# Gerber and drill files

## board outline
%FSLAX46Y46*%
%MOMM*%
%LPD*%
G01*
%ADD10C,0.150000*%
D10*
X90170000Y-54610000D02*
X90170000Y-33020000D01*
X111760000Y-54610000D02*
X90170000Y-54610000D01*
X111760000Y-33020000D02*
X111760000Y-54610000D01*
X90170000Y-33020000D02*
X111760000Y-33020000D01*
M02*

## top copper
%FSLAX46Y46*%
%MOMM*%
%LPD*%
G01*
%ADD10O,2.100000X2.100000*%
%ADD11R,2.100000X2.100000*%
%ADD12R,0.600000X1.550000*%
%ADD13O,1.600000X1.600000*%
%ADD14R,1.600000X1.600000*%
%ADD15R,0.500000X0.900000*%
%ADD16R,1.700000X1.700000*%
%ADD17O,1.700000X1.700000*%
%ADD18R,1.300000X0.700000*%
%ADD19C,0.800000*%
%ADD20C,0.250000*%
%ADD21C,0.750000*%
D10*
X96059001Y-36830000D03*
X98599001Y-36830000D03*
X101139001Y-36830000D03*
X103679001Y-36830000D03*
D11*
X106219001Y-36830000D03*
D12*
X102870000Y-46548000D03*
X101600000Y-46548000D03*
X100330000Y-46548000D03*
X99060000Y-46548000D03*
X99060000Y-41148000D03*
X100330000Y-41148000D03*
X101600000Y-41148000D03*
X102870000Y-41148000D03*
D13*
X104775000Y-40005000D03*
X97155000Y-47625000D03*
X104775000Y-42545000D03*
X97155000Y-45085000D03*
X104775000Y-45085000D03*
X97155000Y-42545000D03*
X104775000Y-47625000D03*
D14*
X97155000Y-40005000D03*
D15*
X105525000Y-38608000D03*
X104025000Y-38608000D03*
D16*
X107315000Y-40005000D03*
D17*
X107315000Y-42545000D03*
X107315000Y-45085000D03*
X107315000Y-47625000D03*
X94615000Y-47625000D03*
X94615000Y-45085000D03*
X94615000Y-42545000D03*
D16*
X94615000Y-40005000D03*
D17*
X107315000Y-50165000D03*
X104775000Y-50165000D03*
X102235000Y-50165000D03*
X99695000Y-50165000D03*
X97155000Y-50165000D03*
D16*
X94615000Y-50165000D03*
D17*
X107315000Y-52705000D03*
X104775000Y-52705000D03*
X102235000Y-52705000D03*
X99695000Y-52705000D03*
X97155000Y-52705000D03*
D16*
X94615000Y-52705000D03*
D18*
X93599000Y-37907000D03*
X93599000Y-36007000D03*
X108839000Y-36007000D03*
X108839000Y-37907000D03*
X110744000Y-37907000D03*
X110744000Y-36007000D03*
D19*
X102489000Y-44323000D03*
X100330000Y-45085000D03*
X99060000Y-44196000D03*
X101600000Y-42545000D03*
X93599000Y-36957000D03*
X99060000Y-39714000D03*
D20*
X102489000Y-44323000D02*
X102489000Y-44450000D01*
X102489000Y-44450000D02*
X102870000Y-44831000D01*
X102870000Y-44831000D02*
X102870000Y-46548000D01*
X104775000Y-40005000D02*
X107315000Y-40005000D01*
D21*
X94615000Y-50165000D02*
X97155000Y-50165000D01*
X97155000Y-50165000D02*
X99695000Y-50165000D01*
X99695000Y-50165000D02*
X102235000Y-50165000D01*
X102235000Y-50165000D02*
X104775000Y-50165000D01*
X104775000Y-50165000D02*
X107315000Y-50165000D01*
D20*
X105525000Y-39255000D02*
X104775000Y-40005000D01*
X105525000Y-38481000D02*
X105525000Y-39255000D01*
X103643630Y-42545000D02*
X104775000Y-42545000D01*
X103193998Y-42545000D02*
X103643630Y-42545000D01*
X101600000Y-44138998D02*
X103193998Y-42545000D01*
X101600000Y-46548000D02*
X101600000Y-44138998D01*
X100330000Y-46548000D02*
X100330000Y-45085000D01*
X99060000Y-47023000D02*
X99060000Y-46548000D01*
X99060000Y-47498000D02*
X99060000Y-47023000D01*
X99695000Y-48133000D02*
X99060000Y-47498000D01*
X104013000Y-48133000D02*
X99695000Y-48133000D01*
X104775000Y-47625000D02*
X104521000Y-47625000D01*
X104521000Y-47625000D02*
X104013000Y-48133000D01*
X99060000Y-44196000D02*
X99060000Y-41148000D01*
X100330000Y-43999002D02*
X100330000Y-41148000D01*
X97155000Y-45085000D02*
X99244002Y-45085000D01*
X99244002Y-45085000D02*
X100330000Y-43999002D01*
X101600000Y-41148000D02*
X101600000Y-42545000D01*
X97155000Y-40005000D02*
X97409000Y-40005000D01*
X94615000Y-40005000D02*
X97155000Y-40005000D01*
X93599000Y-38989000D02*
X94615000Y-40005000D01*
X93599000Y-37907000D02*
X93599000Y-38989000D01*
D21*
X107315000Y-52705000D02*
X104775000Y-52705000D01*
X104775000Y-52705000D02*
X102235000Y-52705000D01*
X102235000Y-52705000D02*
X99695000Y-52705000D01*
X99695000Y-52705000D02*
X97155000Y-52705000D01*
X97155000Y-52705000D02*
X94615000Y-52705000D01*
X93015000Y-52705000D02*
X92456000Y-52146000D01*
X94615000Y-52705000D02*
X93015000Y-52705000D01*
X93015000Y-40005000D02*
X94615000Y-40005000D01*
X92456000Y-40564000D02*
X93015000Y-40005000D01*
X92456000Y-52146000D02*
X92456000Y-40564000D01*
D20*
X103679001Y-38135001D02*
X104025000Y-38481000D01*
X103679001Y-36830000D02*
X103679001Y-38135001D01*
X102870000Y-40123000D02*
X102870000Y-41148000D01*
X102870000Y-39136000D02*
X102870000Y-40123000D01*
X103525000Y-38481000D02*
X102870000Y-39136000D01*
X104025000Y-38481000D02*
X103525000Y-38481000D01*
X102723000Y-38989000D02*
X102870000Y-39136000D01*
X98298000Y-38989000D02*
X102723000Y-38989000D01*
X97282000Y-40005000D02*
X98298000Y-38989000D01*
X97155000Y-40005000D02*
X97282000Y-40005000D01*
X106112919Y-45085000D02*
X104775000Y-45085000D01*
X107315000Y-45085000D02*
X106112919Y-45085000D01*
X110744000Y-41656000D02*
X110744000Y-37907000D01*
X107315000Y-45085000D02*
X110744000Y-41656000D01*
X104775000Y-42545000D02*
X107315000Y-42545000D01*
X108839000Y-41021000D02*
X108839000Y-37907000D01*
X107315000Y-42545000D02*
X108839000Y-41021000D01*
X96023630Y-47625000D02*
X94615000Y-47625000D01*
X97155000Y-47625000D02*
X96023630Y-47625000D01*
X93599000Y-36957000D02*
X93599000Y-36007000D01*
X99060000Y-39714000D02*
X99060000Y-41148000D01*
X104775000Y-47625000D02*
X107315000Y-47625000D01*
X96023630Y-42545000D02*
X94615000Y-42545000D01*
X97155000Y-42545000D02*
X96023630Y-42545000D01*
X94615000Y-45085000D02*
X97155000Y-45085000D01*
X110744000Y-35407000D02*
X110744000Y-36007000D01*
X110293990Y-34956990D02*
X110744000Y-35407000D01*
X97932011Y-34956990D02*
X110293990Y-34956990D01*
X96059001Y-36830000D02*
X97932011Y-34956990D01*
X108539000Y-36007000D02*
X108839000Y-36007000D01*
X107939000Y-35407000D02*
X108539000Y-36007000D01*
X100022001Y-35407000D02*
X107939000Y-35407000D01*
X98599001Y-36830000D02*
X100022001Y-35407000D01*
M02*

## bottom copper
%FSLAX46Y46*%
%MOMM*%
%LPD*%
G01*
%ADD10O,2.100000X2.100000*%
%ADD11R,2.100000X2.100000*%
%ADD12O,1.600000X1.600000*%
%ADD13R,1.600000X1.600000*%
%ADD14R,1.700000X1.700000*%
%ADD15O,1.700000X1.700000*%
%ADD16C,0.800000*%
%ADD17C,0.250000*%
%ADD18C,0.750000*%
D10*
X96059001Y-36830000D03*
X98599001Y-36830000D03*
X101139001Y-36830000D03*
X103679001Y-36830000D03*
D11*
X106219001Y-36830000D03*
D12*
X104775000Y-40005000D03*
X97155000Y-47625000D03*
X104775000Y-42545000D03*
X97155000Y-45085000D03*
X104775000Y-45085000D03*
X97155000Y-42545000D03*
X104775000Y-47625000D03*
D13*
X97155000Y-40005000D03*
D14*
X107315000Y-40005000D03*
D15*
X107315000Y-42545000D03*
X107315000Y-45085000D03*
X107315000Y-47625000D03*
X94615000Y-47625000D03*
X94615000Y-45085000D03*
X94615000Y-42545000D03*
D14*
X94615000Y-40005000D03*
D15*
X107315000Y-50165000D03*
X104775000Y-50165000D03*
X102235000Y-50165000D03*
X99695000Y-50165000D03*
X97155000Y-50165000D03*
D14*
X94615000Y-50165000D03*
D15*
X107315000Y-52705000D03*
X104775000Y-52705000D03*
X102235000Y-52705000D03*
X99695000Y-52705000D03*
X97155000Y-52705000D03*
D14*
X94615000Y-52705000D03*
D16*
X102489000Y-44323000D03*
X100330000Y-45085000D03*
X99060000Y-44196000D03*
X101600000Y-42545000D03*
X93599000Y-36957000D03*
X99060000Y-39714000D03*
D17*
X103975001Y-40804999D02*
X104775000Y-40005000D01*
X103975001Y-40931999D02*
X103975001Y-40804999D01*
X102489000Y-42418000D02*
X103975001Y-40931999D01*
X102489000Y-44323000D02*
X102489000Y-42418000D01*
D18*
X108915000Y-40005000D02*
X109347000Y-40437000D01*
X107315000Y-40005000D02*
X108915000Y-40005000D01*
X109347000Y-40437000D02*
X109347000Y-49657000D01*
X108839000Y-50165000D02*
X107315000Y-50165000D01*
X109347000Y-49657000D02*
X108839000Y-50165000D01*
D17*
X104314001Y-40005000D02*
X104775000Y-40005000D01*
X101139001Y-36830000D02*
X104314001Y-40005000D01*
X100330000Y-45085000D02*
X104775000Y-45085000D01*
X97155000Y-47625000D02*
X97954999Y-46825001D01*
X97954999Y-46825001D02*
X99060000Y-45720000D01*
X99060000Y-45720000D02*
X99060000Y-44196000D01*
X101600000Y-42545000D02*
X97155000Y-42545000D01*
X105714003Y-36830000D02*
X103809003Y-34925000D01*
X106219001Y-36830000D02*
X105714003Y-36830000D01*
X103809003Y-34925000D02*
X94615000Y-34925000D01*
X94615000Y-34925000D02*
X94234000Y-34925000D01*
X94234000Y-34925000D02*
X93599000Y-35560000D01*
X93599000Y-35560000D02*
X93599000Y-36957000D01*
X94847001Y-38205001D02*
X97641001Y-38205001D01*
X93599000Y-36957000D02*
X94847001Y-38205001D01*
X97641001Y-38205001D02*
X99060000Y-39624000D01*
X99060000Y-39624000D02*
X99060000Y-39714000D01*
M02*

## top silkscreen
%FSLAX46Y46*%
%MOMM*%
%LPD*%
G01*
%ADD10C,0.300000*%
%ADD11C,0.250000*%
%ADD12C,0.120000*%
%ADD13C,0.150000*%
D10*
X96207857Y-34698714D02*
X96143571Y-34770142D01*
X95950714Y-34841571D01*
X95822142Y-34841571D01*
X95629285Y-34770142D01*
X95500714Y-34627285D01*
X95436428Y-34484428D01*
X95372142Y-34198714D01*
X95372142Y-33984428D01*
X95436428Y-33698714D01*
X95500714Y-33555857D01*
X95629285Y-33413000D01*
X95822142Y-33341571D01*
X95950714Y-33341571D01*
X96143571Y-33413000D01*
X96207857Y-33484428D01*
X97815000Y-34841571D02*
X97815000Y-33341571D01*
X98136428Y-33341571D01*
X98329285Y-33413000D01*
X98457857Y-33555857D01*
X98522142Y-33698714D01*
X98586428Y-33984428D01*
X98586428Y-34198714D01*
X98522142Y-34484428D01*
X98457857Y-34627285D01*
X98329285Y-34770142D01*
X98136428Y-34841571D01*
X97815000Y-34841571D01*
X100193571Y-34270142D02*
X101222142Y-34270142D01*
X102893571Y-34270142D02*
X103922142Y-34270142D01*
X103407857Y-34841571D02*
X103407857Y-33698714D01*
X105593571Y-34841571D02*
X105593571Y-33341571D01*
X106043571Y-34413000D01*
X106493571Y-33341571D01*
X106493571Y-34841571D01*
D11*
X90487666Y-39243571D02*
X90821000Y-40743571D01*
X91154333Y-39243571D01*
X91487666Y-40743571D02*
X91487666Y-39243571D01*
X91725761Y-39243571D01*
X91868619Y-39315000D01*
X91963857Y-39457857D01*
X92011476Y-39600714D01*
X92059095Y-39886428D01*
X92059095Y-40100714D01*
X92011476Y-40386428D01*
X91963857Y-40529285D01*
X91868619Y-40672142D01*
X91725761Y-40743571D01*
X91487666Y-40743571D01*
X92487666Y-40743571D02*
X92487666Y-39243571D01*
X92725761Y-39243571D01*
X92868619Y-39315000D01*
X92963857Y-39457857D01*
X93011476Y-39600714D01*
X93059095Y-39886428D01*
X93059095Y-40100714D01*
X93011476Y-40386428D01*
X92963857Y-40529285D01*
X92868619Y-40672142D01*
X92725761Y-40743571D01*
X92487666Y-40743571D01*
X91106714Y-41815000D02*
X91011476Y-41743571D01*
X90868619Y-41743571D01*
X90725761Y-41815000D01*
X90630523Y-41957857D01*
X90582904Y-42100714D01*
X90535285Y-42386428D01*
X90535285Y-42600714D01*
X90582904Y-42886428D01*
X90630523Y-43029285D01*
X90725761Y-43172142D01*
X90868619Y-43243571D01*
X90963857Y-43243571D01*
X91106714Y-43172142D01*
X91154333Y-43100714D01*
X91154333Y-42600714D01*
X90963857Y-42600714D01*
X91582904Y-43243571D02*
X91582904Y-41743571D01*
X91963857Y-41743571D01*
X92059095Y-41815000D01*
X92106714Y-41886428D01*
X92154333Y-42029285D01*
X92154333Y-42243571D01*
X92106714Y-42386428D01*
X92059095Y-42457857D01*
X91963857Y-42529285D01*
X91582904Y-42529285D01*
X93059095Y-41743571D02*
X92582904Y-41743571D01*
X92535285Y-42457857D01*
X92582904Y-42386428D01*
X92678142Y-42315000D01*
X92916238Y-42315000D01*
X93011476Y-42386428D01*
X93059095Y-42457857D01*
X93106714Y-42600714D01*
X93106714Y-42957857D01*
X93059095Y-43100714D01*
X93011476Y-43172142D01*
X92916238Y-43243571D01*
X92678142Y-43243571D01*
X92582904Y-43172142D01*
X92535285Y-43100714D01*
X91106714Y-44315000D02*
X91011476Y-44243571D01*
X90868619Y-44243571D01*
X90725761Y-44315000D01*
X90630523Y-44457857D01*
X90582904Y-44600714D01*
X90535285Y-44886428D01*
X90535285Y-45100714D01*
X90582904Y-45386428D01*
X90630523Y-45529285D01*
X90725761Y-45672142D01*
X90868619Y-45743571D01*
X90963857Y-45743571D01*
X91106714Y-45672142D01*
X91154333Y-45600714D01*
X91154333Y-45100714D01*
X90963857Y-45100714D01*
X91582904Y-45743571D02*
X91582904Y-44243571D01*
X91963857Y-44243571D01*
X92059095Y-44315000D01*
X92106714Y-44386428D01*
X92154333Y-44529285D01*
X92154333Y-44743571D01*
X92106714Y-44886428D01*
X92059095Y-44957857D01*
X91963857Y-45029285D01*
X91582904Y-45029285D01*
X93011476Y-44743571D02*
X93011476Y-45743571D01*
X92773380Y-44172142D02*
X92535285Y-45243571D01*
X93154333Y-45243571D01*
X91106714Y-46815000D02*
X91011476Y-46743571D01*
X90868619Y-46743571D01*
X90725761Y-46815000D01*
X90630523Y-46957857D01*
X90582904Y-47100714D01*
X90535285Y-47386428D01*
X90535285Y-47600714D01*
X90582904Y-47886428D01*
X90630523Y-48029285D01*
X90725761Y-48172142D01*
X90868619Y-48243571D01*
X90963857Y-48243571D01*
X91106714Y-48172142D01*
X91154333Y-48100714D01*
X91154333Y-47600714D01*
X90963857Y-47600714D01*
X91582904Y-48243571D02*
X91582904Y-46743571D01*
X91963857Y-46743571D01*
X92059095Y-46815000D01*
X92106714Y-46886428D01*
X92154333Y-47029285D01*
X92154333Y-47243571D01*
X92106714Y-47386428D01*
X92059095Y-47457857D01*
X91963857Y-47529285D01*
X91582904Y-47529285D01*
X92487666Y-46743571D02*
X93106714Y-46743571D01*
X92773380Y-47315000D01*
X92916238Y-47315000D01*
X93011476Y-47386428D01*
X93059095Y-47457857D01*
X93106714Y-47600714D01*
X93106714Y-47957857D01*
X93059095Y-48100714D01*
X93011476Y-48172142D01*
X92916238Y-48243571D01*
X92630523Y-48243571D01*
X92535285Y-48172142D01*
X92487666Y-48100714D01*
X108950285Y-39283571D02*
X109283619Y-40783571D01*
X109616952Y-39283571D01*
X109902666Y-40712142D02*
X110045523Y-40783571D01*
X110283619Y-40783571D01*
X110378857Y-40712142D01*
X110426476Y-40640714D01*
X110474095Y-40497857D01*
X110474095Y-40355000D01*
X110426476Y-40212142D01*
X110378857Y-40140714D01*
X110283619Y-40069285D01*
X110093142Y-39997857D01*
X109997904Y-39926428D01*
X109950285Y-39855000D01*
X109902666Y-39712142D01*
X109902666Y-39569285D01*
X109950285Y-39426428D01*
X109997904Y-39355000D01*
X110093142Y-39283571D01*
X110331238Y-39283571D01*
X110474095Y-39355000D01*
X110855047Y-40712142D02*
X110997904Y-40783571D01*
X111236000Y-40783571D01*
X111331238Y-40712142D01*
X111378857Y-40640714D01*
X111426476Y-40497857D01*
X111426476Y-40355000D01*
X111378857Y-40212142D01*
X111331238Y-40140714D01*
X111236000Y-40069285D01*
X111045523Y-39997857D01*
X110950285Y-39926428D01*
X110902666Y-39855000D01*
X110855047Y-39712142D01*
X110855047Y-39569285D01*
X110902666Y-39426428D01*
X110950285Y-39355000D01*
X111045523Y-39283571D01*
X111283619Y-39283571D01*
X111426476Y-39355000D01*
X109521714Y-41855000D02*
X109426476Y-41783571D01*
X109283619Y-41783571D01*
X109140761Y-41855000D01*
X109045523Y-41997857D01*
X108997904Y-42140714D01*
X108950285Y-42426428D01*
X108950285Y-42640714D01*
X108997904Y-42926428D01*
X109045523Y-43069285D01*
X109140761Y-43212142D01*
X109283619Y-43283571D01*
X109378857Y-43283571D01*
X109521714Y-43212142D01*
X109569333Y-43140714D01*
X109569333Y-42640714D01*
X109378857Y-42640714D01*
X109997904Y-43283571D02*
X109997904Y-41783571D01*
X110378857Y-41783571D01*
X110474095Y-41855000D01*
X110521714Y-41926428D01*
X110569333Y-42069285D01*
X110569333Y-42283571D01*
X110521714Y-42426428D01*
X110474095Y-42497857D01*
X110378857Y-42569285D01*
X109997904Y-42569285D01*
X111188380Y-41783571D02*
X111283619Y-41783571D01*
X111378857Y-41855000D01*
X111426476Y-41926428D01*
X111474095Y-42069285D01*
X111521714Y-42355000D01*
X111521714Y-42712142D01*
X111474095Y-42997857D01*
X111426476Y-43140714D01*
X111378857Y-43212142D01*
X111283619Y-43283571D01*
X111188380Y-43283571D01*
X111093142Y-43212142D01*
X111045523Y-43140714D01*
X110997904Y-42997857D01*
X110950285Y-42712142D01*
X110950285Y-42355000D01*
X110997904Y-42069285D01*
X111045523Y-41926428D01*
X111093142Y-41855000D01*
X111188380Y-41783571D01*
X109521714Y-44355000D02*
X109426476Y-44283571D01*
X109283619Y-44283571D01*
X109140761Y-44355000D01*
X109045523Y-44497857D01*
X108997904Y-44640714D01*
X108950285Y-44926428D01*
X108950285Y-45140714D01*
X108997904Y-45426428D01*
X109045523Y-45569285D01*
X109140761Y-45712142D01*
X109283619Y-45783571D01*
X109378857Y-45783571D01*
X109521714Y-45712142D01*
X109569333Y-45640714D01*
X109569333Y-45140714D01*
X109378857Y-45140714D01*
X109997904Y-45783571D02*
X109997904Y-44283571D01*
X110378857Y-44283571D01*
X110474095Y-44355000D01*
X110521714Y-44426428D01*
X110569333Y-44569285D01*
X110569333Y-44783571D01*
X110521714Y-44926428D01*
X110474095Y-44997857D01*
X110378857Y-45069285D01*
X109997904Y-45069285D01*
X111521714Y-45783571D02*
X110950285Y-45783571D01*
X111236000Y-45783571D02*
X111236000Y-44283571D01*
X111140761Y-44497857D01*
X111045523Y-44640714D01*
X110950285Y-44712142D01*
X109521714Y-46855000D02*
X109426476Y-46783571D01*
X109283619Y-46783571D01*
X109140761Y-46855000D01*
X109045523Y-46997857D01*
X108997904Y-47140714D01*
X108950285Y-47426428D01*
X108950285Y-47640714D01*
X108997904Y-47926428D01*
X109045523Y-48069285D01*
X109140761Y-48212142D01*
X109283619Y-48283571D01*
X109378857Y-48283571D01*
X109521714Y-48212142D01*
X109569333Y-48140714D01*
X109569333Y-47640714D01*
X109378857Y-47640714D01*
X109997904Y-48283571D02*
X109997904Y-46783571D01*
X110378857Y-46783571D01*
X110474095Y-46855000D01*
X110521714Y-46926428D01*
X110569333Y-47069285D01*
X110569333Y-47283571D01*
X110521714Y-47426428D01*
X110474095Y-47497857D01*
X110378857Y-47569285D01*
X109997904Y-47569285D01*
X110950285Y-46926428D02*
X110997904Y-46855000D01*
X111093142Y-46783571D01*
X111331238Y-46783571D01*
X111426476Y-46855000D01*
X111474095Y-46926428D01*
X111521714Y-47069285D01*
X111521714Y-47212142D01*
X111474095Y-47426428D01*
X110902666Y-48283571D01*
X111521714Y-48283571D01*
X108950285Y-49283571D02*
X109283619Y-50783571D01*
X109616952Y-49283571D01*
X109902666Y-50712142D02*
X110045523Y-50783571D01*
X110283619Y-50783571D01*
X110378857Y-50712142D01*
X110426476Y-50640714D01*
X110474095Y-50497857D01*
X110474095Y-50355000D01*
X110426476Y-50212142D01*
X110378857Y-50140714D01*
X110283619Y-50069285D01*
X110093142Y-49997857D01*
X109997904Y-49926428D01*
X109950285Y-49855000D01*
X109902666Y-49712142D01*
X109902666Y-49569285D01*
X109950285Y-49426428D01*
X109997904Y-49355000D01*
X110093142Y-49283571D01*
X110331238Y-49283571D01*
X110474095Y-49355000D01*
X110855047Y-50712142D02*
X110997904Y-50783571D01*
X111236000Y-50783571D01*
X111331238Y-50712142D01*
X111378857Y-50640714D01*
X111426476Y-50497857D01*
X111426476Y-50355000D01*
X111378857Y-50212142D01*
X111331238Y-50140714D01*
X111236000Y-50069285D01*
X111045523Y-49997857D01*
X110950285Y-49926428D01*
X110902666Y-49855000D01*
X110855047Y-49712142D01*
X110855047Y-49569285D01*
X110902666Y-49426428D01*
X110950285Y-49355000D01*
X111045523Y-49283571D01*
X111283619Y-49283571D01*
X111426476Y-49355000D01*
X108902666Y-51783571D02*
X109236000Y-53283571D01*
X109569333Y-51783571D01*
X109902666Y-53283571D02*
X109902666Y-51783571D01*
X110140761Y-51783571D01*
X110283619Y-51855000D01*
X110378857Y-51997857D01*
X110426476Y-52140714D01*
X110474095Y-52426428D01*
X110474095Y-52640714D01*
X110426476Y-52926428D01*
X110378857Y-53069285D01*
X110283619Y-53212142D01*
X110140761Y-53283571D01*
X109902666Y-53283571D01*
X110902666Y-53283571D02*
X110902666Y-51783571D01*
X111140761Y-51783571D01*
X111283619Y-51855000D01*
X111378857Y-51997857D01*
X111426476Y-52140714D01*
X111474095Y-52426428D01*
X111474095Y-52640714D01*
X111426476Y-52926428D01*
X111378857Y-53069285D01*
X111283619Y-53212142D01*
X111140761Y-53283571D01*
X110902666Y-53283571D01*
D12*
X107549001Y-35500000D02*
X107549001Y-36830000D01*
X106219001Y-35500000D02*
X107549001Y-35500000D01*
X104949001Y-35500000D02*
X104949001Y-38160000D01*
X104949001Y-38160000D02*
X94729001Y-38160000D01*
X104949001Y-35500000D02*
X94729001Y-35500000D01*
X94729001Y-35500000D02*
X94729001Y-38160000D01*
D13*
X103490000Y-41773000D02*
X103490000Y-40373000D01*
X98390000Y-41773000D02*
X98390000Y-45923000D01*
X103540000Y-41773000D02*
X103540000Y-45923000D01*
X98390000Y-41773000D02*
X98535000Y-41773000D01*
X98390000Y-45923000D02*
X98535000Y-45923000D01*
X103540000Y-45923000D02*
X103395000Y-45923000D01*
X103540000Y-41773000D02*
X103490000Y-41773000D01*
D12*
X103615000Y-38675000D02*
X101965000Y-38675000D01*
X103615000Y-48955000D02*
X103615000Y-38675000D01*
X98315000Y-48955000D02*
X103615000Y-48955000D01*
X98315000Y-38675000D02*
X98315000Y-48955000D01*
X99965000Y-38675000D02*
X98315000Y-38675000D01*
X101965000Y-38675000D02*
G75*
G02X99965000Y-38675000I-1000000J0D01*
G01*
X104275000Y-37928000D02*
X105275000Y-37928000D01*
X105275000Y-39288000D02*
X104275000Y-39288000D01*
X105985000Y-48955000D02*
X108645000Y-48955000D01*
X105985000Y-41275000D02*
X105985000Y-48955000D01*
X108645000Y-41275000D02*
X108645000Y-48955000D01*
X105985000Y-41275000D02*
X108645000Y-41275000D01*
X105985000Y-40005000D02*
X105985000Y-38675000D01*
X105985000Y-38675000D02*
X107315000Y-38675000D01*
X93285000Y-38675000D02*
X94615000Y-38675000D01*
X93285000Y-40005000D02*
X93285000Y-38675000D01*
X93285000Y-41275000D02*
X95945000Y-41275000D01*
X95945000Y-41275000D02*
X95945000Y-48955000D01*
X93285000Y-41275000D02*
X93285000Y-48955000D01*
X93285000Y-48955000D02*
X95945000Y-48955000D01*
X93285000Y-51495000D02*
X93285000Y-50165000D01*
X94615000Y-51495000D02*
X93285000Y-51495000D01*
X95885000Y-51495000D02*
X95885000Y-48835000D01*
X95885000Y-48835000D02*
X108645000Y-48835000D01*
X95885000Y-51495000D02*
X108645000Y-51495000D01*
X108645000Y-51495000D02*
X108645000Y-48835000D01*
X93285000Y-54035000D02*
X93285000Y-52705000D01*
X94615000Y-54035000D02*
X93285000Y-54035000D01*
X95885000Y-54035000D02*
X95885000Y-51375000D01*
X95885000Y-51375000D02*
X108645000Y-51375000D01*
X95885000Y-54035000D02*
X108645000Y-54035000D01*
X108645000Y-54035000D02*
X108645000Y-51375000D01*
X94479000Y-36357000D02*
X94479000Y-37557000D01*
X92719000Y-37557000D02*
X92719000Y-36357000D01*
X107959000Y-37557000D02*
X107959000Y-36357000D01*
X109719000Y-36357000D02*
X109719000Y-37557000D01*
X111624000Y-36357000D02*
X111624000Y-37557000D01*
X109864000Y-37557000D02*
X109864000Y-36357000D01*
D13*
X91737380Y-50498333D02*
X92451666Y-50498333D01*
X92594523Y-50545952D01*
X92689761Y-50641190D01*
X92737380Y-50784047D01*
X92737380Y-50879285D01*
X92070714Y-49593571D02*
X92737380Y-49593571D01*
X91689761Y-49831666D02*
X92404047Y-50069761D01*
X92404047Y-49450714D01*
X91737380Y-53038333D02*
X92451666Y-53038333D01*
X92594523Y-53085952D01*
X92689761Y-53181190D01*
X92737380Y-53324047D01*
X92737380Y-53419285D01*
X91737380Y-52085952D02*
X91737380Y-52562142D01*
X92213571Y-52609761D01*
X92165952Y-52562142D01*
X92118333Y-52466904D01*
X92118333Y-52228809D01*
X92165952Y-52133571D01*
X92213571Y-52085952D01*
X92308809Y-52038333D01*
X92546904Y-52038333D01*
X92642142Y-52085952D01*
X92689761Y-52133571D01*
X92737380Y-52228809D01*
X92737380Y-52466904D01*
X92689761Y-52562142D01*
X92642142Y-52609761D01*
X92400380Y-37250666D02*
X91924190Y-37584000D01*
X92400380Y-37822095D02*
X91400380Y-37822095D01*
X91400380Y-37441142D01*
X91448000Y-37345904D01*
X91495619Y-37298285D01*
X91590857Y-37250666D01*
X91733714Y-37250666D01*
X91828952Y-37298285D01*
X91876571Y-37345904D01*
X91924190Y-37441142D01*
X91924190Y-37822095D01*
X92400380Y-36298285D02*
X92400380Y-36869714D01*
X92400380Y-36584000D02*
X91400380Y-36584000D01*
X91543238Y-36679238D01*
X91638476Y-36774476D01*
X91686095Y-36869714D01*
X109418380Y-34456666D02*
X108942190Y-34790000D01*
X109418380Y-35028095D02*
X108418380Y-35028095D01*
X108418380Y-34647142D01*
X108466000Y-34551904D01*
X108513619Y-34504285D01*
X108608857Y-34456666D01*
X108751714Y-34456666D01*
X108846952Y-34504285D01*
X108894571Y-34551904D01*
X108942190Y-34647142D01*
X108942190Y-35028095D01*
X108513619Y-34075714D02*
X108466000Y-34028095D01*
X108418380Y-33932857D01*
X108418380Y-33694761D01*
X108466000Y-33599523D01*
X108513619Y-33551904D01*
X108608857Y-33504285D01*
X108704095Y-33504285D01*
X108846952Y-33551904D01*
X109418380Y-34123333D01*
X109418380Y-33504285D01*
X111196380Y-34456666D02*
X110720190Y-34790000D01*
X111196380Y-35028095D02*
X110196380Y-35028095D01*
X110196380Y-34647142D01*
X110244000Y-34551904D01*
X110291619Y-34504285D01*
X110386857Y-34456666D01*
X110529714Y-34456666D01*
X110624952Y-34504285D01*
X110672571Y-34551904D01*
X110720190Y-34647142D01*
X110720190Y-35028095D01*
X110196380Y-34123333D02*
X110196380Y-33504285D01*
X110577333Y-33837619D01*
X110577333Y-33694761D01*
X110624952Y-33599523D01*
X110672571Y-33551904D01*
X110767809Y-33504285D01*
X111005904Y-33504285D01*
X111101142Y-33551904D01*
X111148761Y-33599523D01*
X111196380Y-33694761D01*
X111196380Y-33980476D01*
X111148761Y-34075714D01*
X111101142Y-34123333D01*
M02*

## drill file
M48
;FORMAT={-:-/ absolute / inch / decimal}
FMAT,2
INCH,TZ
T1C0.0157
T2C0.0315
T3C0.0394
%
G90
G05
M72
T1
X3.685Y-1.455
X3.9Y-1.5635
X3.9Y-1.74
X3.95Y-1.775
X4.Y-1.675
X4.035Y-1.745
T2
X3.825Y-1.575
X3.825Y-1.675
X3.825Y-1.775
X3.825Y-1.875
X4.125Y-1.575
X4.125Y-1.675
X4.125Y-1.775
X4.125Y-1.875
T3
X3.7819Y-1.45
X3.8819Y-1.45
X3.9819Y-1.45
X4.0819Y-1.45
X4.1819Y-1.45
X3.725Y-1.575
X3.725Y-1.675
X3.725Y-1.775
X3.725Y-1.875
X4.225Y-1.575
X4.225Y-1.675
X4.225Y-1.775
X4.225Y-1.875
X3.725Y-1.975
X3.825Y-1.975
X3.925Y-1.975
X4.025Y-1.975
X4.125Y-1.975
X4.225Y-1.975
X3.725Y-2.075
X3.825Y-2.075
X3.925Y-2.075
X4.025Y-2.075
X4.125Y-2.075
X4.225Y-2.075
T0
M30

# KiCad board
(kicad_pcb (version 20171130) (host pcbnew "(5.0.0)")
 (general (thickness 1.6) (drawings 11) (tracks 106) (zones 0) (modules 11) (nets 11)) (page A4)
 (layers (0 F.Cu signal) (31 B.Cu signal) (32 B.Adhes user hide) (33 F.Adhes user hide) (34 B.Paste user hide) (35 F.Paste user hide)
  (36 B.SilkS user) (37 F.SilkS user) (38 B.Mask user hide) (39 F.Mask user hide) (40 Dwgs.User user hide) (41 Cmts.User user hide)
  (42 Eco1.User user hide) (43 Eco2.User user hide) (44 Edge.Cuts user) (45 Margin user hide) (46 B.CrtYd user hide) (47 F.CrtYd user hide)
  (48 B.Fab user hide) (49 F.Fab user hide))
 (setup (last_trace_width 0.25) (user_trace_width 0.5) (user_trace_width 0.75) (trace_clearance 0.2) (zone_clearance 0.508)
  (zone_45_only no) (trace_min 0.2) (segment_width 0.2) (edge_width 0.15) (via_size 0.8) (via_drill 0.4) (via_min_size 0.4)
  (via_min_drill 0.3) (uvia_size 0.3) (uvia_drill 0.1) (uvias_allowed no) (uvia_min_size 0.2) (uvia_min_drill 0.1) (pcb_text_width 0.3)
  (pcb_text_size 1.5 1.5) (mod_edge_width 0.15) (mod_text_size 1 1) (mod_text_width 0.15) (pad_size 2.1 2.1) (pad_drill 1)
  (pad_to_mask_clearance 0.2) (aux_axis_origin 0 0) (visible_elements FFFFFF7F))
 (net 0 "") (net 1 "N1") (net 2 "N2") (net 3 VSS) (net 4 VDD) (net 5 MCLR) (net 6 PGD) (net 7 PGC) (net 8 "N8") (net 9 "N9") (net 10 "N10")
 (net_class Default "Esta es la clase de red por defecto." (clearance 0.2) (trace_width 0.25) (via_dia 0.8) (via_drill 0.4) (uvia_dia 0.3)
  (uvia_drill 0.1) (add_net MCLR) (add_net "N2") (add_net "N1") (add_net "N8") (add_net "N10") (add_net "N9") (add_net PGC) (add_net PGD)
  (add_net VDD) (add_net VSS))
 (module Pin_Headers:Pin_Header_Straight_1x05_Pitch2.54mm (layer F.Cu) (at 106.219001 36.83 270)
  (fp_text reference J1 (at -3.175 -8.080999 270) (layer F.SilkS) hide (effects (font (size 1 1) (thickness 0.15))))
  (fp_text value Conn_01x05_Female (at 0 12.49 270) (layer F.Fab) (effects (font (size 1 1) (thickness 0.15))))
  (fp_line (start -1.33 -1.33) (end 0 -1.33) (layer F.SilkS) (width 0.12))
  (fp_line (start -1.33 0) (end -1.33 -1.33) (layer F.SilkS) (width 0.12))
  (fp_line (start -1.33 1.27) (end 1.33 1.27) (layer F.SilkS) (width 0.12))
  (fp_line (start 1.33 1.27) (end 1.33 11.49) (layer F.SilkS) (width 0.12))
  (fp_line (start -1.33 1.27) (end -1.33 11.49) (layer F.SilkS) (width 0.12))
  (fp_line (start -1.33 11.49) (end 1.33 11.49) (layer F.SilkS) (width 0.12))
  (pad 5 thru_hole oval (at 0 10.16 270) (size 2.1 2.1) (drill 1) (layers *.Cu *.Mask) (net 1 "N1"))
  (pad 4 thru_hole oval (at 0 7.62 270) (size 2.1 2.1) (drill 1) (layers *.Cu *.Mask) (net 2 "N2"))
  (pad 3 thru_hole oval (at 0 5.08 270) (size 2.1 2.1) (drill 1) (layers *.Cu *.Mask) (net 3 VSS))
  (pad 2 thru_hole oval (at 0 2.54 270) (size 2.1 2.1) (drill 1) (layers *.Cu *.Mask) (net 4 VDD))
  (pad 1 thru_hole rect (at 0 0 270) (size 2.1 2.1) (drill 1) (layers *.Cu *.Mask) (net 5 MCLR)))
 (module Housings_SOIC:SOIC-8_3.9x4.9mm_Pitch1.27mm (layer F.Cu) (at 100.965 43.848 270)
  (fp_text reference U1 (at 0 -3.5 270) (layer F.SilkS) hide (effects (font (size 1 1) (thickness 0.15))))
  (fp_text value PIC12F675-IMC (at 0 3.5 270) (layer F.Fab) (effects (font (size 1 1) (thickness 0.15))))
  (fp_line (start -2.075 -2.525) (end -3.475 -2.525) (layer F.SilkS) (width 0.15))
  (fp_line (start -2.075 2.575) (end 2.075 2.575) (layer F.SilkS) (width 0.15))
  (fp_line (start -2.075 -2.575) (end 2.075 -2.575) (layer F.SilkS) (width 0.15))
  (fp_line (start -2.075 2.575) (end -2.075 2.43) (layer F.SilkS) (width 0.15))
  (fp_line (start 2.075 2.575) (end 2.075 2.43) (layer F.SilkS) (width 0.15))
  (fp_line (start 2.075 -2.575) (end 2.075 -2.43) (layer F.SilkS) (width 0.15))
  (fp_line (start -2.075 -2.575) (end -2.075 -2.525) (layer F.SilkS) (width 0.15))
  (pad 8 smd rect (at 2.7 -1.905 270) (size 1.55 0.6) (layers F.Cu F.Paste F.Mask) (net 3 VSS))
  (pad 7 smd rect (at 2.7 -0.635 270) (size 1.55 0.6) (layers F.Cu F.Paste F.Mask) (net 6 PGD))
  (pad 6 smd rect (at 2.7 0.635 270) (size 1.55 0.6) (layers F.Cu F.Paste F.Mask) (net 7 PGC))
  (pad 5 smd rect (at 2.7 1.905 270) (size 1.55 0.6) (layers F.Cu F.Paste F.Mask) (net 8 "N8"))
  (pad 4 smd rect (at -2.7 1.905 270) (size 1.55 0.6) (layers F.Cu F.Paste F.Mask) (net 5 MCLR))
  (pad 3 smd rect (at -2.7 0.635 270) (size 1.55 0.6) (layers F.Cu F.Paste F.Mask) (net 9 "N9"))
  (pad 2 smd rect (at -2.7 -0.635 270) (size 1.55 0.6) (layers F.Cu F.Paste F.Mask) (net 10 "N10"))
  (pad 1 smd rect (at -2.7 -1.905 270) (size 1.55 0.6) (layers F.Cu F.Paste F.Mask) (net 4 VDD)))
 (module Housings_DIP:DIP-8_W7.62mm (layer F.Cu) (at 97.155 40.005)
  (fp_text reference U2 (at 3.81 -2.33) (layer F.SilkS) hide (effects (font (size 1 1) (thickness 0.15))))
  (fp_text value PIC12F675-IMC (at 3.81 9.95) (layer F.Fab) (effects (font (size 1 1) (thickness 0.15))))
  (fp_line (start 6.46 -1.33) (end 4.81 -1.33) (layer F.SilkS) (width 0.12))
  (fp_line (start 6.46 8.95) (end 6.46 -1.33) (layer F.SilkS) (width 0.12))
  (fp_line (start 1.16 8.95) (end 6.46 8.95) (layer F.SilkS) (width 0.12))
  (fp_line (start 1.16 -1.33) (end 1.16 8.95) (layer F.SilkS) (width 0.12))
  (fp_line (start 2.81 -1.33) (end 1.16 -1.33) (layer F.SilkS) (width 0.12))
  (fp_arc (start 3.81 -1.33) (end 2.81 -1.33) (angle -180) (layer F.SilkS) (width 0.12))
  (pad 8 thru_hole oval (at 7.62 0) (size 1.6 1.6) (drill 0.8) (layers *.Cu *.Mask) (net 3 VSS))
  (pad 4 thru_hole oval (at 0 7.62) (size 1.6 1.6) (drill 0.8) (layers *.Cu *.Mask) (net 5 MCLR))
  (pad 7 thru_hole oval (at 7.62 2.54) (size 1.6 1.6) (drill 0.8) (layers *.Cu *.Mask) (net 6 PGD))
  (pad 3 thru_hole oval (at 0 5.08) (size 1.6 1.6) (drill 0.8) (layers *.Cu *.Mask) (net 9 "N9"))
  (pad 6 thru_hole oval (at 7.62 5.08) (size 1.6 1.6) (drill 0.8) (layers *.Cu *.Mask) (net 7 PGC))
  (pad 2 thru_hole oval (at 0 2.54) (size 1.6 1.6) (drill 0.8) (layers *.Cu *.Mask) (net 10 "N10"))
  (pad 5 thru_hole oval (at 7.62 7.62) (size 1.6 1.6) (drill 0.8) (layers *.Cu *.Mask) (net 8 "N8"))
  (pad 1 thru_hole rect (at 0 0) (size 1.6 1.6) (drill 0.8) (layers *.Cu *.Mask) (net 4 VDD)))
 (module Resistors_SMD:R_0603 (layer F.Cu) (at 104.775 38.608)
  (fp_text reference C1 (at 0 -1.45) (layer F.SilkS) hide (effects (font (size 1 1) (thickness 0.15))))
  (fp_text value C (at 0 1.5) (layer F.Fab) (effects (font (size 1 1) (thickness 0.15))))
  (fp_line (start -0.5 -0.68) (end 0.5 -0.68) (layer F.SilkS) (width 0.12))
  (fp_line (start 0.5 0.68) (end -0.5 0.68) (layer F.SilkS) (width 0.12))
  (pad 2 smd rect (at 0.75 0) (size 0.5 0.9) (layers F.Cu F.Paste F.Mask) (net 3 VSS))
  (pad 1 smd rect (at -0.75 0) (size 0.5 0.9) (layers F.Cu F.Paste F.Mask) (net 4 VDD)))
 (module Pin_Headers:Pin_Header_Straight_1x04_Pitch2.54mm (layer F.Cu) (at 107.315 40.005)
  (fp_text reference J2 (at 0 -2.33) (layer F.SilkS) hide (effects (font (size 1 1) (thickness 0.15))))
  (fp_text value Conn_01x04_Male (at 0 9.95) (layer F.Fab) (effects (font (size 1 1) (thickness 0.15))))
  (fp_line (start -1.33 8.95) (end 1.33 8.95) (layer F.SilkS) (width 0.12))
  (fp_line (start -1.33 1.27) (end -1.33 8.95) (layer F.SilkS) (width 0.12))
  (fp_line (start 1.33 1.27) (end 1.33 8.95) (layer F.SilkS) (width 0.12))
  (fp_line (start -1.33 1.27) (end 1.33 1.27) (layer F.SilkS) (width 0.12))
  (fp_line (start -1.33 0) (end -1.33 -1.33) (layer F.SilkS) (width 0.12))
  (fp_line (start -1.33 -1.33) (end 0 -1.33) (layer F.SilkS) (width 0.12))
  (pad 1 thru_hole rect (at 0 0) (size 1.7 1.7) (drill 1) (layers *.Cu *.Mask) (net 3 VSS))
  (pad 2 thru_hole oval (at 0 2.54) (size 1.7 1.7) (drill 1) (layers *.Cu *.Mask) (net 6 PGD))
  (pad 3 thru_hole oval (at 0 5.08) (size 1.7 1.7) (drill 1) (layers *.Cu *.Mask) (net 7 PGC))
  (pad 4 thru_hole oval (at 0 7.62) (size 1.7 1.7) (drill 1) (layers *.Cu *.Mask) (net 8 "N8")))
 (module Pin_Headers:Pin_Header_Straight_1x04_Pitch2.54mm (layer F.Cu) (at 94.615 40.005)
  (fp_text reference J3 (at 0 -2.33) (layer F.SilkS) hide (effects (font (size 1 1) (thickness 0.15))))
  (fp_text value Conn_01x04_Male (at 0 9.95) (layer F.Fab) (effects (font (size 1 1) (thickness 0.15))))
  (fp_line (start -1.33 -1.33) (end 0 -1.33) (layer F.SilkS) (width 0.12))
  (fp_line (start -1.33 0) (end -1.33 -1.33) (layer F.SilkS) (width 0.12))
  (fp_line (start -1.33 1.27) (end 1.33 1.27) (layer F.SilkS) (width 0.12))
  (fp_line (start 1.33 1.27) (end 1.33 8.95) (layer F.SilkS) (width 0.12))
  (fp_line (start -1.33 1.27) (end -1.33 8.95) (layer F.SilkS) (width 0.12))
  (fp_line (start -1.33 8.95) (end 1.33 8.95) (layer F.SilkS) (width 0.12))
  (pad 4 thru_hole oval (at 0 7.62) (size 1.7 1.7) (drill 1) (layers *.Cu *.Mask) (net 5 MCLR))
  (pad 3 thru_hole oval (at 0 5.08) (size 1.7 1.7) (drill 1) (layers *.Cu *.Mask) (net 9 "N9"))
  (pad 2 thru_hole oval (at 0 2.54) (size 1.7 1.7) (drill 1) (layers *.Cu *.Mask) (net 10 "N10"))
  (pad 1 thru_hole rect (at 0 0) (size 1.7 1.7) (drill 1) (layers *.Cu *.Mask) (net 4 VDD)))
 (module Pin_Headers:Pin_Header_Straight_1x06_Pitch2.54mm (layer F.Cu) (at 94.615 50.165 90)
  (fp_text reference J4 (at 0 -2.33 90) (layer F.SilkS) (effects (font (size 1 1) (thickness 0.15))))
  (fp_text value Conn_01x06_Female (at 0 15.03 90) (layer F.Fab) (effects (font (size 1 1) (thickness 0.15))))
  (fp_line (start -1.33 -1.33) (end 0 -1.33) (layer F.SilkS) (width 0.12))
  (fp_line (start -1.33 0) (end -1.33 -1.33) (layer F.SilkS) (width 0.12))
  (fp_line (start -1.33 1.27) (end 1.33 1.27) (layer F.SilkS) (width 0.12))
  (fp_line (start 1.33 1.27) (end 1.33 14.03) (layer F.SilkS) (width 0.12))
  (fp_line (start -1.33 1.27) (end -1.33 14.03) (layer F.SilkS) (width 0.12))
  (fp_line (start -1.33 14.03) (end 1.33 14.03) (layer F.SilkS) (width 0.12))
  (pad 6 thru_hole oval (at 0 12.7 90) (size 1.7 1.7) (drill 1) (layers *.Cu *.Mask) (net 3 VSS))
  (pad 5 thru_hole oval (at 0 10.16 90) (size 1.7 1.7) (drill 1) (layers *.Cu *.Mask) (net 3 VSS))
  (pad 4 thru_hole oval (at 0 7.62 90) (size 1.7 1.7) (drill 1) (layers *.Cu *.Mask) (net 3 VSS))
  (pad 3 thru_hole oval (at 0 5.08 90) (size 1.7 1.7) (drill 1) (layers *.Cu *.Mask) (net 3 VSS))
  (pad 2 thru_hole oval (at 0 2.54 90) (size 1.7 1.7) (drill 1) (layers *.Cu *.Mask) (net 3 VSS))
  (pad 1 thru_hole rect (at 0 0 90) (size 1.7 1.7) (drill 1) (layers *.Cu *.Mask) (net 3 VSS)))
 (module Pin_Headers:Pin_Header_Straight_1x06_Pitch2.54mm (layer F.Cu) (at 94.615 52.705 90)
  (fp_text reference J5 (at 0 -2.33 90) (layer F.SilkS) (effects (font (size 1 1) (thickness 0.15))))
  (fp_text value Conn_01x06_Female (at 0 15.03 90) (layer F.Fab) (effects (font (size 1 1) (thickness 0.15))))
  (fp_line (start -1.33 -1.33) (end 0 -1.33) (layer F.SilkS) (width 0.12))
  (fp_line (start -1.33 0) (end -1.33 -1.33) (layer F.SilkS) (width 0.12))
  (fp_line (start -1.33 1.27) (end 1.33 1.27) (layer F.SilkS) (width 0.12))
  (fp_line (start 1.33 1.27) (end 1.33 14.03) (layer F.SilkS) (width 0.12))
  (fp_line (start -1.33 1.27) (end -1.33 14.03) (layer F.SilkS) (width 0.12))
  (fp_line (start -1.33 14.03) (end 1.33 14.03) (layer F.SilkS) (width 0.12))
  (pad 6 thru_hole oval (at 0 12.7 90) (size 1.7 1.7) (drill 1) (layers *.Cu *.Mask) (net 4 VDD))
  (pad 5 thru_hole oval (at 0 10.16 90) (size 1.7 1.7) (drill 1) (layers *.Cu *.Mask) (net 4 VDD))
  (pad 4 thru_hole oval (at 0 7.62 90) (size 1.7 1.7) (drill 1) (layers *.Cu *.Mask) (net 4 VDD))
  (pad 3 thru_hole oval (at 0 5.08 90) (size 1.7 1.7) (drill 1) (layers *.Cu *.Mask) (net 4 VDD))
  (pad 2 thru_hole oval (at 0 2.54 90) (size 1.7 1.7) (drill 1) (layers *.Cu *.Mask) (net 4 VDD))
  (pad 1 thru_hole rect (at 0 0 90) (size 1.7 1.7) (drill 1) (layers *.Cu *.Mask) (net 4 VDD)))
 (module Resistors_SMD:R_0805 (layer F.Cu) (at 93.599 36.957 270)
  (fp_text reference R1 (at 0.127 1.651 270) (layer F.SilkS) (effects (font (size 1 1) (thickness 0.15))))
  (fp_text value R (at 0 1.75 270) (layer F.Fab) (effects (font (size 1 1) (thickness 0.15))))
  (fp_line (start -0.6 -0.88) (end 0.6 -0.88) (layer F.SilkS) (width 0.12))
  (fp_line (start 0.6 0.88) (end -0.6 0.88) (layer F.SilkS) (width 0.12))
  (pad 2 smd rect (at 0.95 0 270) (size 0.7 1.3) (layers F.Cu F.Paste F.Mask) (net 4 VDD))
  (pad 1 smd rect (at -0.95 0 270) (size 0.7 1.3) (layers F.Cu F.Paste F.Mask) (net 5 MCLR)))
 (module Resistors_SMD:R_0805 (layer F.Cu) (at 108.839 36.957 270)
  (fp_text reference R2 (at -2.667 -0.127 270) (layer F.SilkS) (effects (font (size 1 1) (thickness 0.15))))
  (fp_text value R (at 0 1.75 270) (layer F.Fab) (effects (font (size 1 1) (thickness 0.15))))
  (fp_line (start 0.6 0.88) (end -0.6 0.88) (layer F.SilkS) (width 0.12))
  (fp_line (start -0.6 -0.88) (end 0.6 -0.88) (layer F.SilkS) (width 0.12))
  (pad 1 smd rect (at -0.95 0 270) (size 0.7 1.3) (layers F.Cu F.Paste F.Mask) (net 2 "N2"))
  (pad 2 smd rect (at 0.95 0 270) (size 0.7 1.3) (layers F.Cu F.Paste F.Mask) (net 6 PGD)))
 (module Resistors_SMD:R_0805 (layer F.Cu) (at 110.744 36.957 270)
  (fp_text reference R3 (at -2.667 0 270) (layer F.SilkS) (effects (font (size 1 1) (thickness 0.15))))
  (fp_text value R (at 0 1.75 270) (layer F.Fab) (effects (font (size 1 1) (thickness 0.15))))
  (fp_line (start -0.6 -0.88) (end 0.6 -0.88) (layer F.SilkS) (width 0.12))
  (fp_line (start 0.6 0.88) (end -0.6 0.88) (layer F.SilkS) (width 0.12))
  (pad 2 smd rect (at 0.95 0 270) (size 0.7 1.3) (layers F.Cu F.Paste F.Mask) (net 7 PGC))
  (pad 1 smd rect (at -0.95 0 270) (size 0.7 1.3) (layers F.Cu F.Paste F.Mask) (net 1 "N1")))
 (gr_line (start 90.17 54.61) (end 90.17 33.02) (layer Edge.Cuts) (width 0.15))
 (gr_line (start 111.76 54.61) (end 90.17 54.61) (layer Edge.Cuts) (width 0.15))
 (gr_line (start 111.76 33.02) (end 111.76 54.61) (layer Edge.Cuts) (width 0.15))
 (gr_line (start 90.17 33.02) (end 111.76 33.02) (layer Edge.Cuts) (width 0.15))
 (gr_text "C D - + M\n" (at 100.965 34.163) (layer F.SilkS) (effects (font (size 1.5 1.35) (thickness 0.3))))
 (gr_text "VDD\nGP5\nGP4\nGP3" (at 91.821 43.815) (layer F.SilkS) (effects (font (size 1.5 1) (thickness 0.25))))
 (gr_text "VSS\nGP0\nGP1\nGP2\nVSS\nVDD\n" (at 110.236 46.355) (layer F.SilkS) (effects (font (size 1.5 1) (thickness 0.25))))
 (segment (start 103.975001 40.804999) (end 104.775 40.005) (width 0.25) (layer B.Cu) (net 3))
 (segment (start 103.975001 40.931999) (end 103.975001 40.804999) (width 0.25) (layer B.Cu) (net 3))
 (segment (start 102.489 44.323) (end 102.489 44.45) (width 0.25) (layer F.Cu) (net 3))
 (segment (start 102.489 44.45) (end 102.87 44.831) (width 0.25) (layer F.Cu) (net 3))
 (segment (start 102.87 44.831) (end 102.87 46.548) (width 0.25) (layer F.Cu) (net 3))
 (segment (start 102.489 42.418) (end 103.975001 40.931999) (width 0.25) (layer B.Cu) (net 3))
 (segment (start 102.489 44.323) (end 102.489 42.418) (width 0.25) (layer B.Cu) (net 3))
 (via (at 102.489 44.323) (size 0.8) (drill 0.4) (layers F.Cu B.Cu) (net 3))
 (segment (start 104.775 40.005) (end 107.315 40.005) (width 0.25) (layer F.Cu) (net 3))
 (segment (start 94.615 50.165) (end 97.155 50.165) (width 0.75) (layer F.Cu) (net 3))
 (segment (start 97.155 50.165) (end 99.695 50.165) (width 0.75) (layer F.Cu) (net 3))
 (segment (start 99.695 50.165) (end 102.235 50.165) (width 0.75) (layer F.Cu) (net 3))
 (segment (start 102.235 50.165) (end 104.775 50.165) (width 0.75) (layer F.Cu) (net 3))
 (segment (start 104.775 50.165) (end 107.315 50.165) (width 0.75) (layer F.Cu) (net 3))
 (segment (start 108.915 40.005) (end 109.347 40.437) (width 0.75) (layer B.Cu) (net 3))
 (segment (start 107.315 40.005) (end 108.915 40.005) (width 0.75) (layer B.Cu) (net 3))
 (segment (start 109.347 40.437) (end 109.347 49.657) (width 0.75) (layer B.Cu) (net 3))
 (segment (start 108.839 50.165) (end 107.315 50.165) (width 0.75) (layer B.Cu) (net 3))
 (segment (start 109.347 49.657) (end 108.839 50.165) (width 0.75) (layer B.Cu) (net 3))
 (segment (start 104.314001 40.005) (end 104.775 40.005) (width 0.25) (layer B.Cu) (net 3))
 (segment (start 101.139001 36.83) (end 104.314001 40.005) (width 0.25) (layer B.Cu) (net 3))
 (segment (start 105.525 39.255) (end 104.775 40.005) (width 0.25) (layer F.Cu) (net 3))
 (segment (start 105.525 38.481) (end 105.525 39.255) (width 0.25) (layer F.Cu) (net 3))
 (segment (start 103.64363 42.545) (end 104.775 42.545) (width 0.25) (layer F.Cu) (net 6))
 (segment (start 103.193998 42.545) (end 103.64363 42.545) (width 0.25) (layer F.Cu) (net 6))
 (segment (start 101.6 44.138998) (end 103.193998 42.545) (width 0.25) (layer F.Cu) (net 6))
 (segment (start 101.6 46.548) (end 101.6 44.138998) (width 0.25) (layer F.Cu) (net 6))
 (via (at 100.33 45.085) (size 0.8) (drill 0.4) (layers F.Cu B.Cu) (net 7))
 (segment (start 100.33 46.548) (end 100.33 45.085) (width 0.25) (layer F.Cu) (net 7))
 (segment (start 100.33 45.085) (end 104.775 45.085) (width 0.25) (layer B.Cu) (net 7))
 (segment (start 99.06 47.023) (end 99.06 46.548) (width 0.25) (layer F.Cu) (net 8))
 (segment (start 99.06 47.498) (end 99.06 47.023) (width 0.25) (layer F.Cu) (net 8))
 (segment (start 99.695 48.133) (end 99.06 47.498) (width 0.25) (layer F.Cu) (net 8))
 (segment (start 104.013 48.133) (end 99.695 48.133) (width 0.25) (layer F.Cu) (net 8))
 (segment (start 104.775 47.625) (end 104.521 47.625) (width 0.25) (layer F.Cu) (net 8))
 (segment (start 104.521 47.625) (end 104.013 48.133) (width 0.25) (layer F.Cu) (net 8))
 (segment (start 97.155 47.625) (end 97.954999 46.825001) (width 0.25) (layer B.Cu) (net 5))
 (segment (start 97.954999 46.825001) (end 99.06 45.72) (width 0.25) (layer B.Cu) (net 5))
 (segment (start 99.06 45.72) (end 99.06 44.196) (width 0.25) (layer B.Cu) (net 5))
 (via (at 99.06 44.196) (size 0.8) (drill 0.4) (layers F.Cu B.Cu) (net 5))
 (segment (start 99.06 44.196) (end 99.06 41.148) (width 0.25) (layer F.Cu) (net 5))
 (segment (start 100.33 43.999002) (end 100.33 41.148) (width 0.25) (layer F.Cu) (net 9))
 (segment (start 97.155 45.085) (end 99.244002 45.085) (width 0.25) (layer F.Cu) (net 9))
 (segment (start 99.244002 45.085) (end 100.33 43.999002) (width 0.25) (layer F.Cu) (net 9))
 (via (at 101.6 42.545) (size 0.8) (drill 0.4) (layers F.Cu B.Cu) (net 10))
 (segment (start 101.6 41.148) (end 101.6 42.545) (width 0.25) (layer F.Cu) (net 10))
 (segment (start 101.6 42.545) (end 97.155 42.545) (width 0.25) (layer B.Cu) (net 10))
 (segment (start 97.155 40.005) (end 97.409 40.005) (width 0.25) (layer F.Cu) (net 4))
 (segment (start 94.615 40.005) (end 97.155 40.005) (width 0.25) (layer F.Cu) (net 4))
 (segment (start 93.599 38.989) (end 94.615 40.005) (width 0.25) (layer F.Cu) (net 4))
 (segment (start 93.599 37.907) (end 93.599 38.989) (width 0.25) (layer F.Cu) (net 4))
 (segment (start 107.315 52.705) (end 104.775 52.705) (width 0.75) (layer F.Cu) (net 4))
 (segment (start 104.775 52.705) (end 102.235 52.705) (width 0.75) (layer F.Cu) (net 4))
 (segment (start 102.235 52.705) (end 99.695 52.705) (width 0.75) (layer F.Cu) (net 4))
 (segment (start 99.695 52.705) (end 97.155 52.705) (width 0.75) (layer F.Cu) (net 4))
 (segment (start 97.155 52.705) (end 94.615 52.705) (width 0.75) (layer F.Cu) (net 4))
 (segment (start 93.015 52.705) (end 92.456 52.146) (width 0.75) (layer F.Cu) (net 4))
 (segment (start 94.615 52.705) (end 93.015 52.705) (width 0.75) (layer F.Cu) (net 4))
 (segment (start 93.015 40.005) (end 94.615 40.005) (width 0.75) (layer F.Cu) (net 4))
 (segment (start 92.456 40.564) (end 93.015 40.005) (width 0.75) (layer F.Cu) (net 4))
 (segment (start 92.456 52.146) (end 92.456 40.564) (width 0.75) (layer F.Cu) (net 4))
 (segment (start 103.679001 38.135001) (end 104.025 38.481) (width 0.25) (layer F.Cu) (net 4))
 (segment (start 103.679001 36.83) (end 103.679001 38.135001) (width 0.25) (layer F.Cu) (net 4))
 (segment (start 102.87 40.123) (end 102.87 41.148) (width 0.25) (layer F.Cu) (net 4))
 (segment (start 102.87 39.136) (end 102.87 40.123) (width 0.25) (layer F.Cu) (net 4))
 (segment (start 103.525 38.481) (end 102.87 39.136) (width 0.25) (layer F.Cu) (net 4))
 (segment (start 104.025 38.481) (end 103.525 38.481) (width 0.25) (layer F.Cu) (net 4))
 (segment (start 102.723 38.989) (end 102.87 39.136) (width 0.25) (layer F.Cu) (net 4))
 (segment (start 98.298 38.989) (end 102.723 38.989) (width 0.25) (layer F.Cu) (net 4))
 (segment (start 97.282 40.005) (end 98.298 38.989) (width 0.25) (layer F.Cu) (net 4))
 (segment (start 97.155 40.005) (end 97.282 40.005) (width 0.25) (layer F.Cu) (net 4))
 (segment (start 106.112919 45.085) (end 104.775 45.085) (width 0.25) (layer F.Cu) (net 7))
 (segment (start 107.315 45.085) (end 106.112919 45.085) (width 0.25) (layer F.Cu) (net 7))
 (segment (start 110.744 41.656) (end 110.744 37.907) (width 0.25) (layer F.Cu) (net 7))
 (segment (start 107.315 45.085) (end 110.744 41.656) (width 0.25) (layer F.Cu) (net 7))
 (segment (start 104.775 42.545) (end 107.315 42.545) (width 0.25) (layer F.Cu) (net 6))
 (segment (start 108.839 41.021) (end 108.839 37.907) (width 0.25) (layer F.Cu) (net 6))
 (segment (start 107.315 42.545) (end 108.839 41.021) (width 0.25) (layer F.Cu) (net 6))
 (segment (start 96.02363 47.625) (end 94.615 47.625) (width 0.25) (layer F.Cu) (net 5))
 (segment (start 97.155 47.625) (end 96.02363 47.625) (width 0.25) (layer F.Cu) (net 5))
 (segment (start 105.714003 36.83) (end 103.809003 34.925) (width 0.25) (layer B.Cu) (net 5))
 (segment (start 106.219001 36.83) (end 105.714003 36.83) (width 0.25) (layer B.Cu) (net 5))
 (segment (start 103.809003 34.925) (end 94.615 34.925) (width 0.25) (layer B.Cu) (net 5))
 (segment (start 94.615 34.925) (end 94.234 34.925) (width 0.25) (layer B.Cu) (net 5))
 (segment (start 94.234 34.925) (end 93.599 35.56) (width 0.25) (layer B.Cu) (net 5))
 (via (at 93.599 36.957) (size 0.8) (drill 0.4) (layers F.Cu B.Cu) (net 5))
 (segment (start 93.599 35.56) (end 93.599 36.957) (width 0.25) (layer B.Cu) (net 5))
 (segment (start 93.599 36.957) (end 93.599 36.007) (width 0.25) (layer F.Cu) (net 5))
 (segment (start 94.847001 38.205001) (end 97.641001 38.205001) (width 0.25) (layer B.Cu) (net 5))
 (segment (start 93.599 36.957) (end 94.847001 38.205001) (width 0.25) (layer B.Cu) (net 5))
 (via (at 99.06 39.714) (size 0.8) (drill 0.4) (layers F.Cu B.Cu) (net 5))
 (segment (start 97.641001 38.205001) (end 99.06 39.624) (width 0.25) (layer B.Cu) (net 5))
 (segment (start 99.06 39.624) (end 99.06 39.714) (width 0.25) (layer B.Cu) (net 5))
 (segment (start 99.06 39.714) (end 99.06 41.148) (width 0.25) (layer F.Cu) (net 5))
 (segment (start 104.775 47.625) (end 107.315 47.625) (width 0.25) (layer F.Cu) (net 8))
 (segment (start 96.02363 42.545) (end 94.615 42.545) (width 0.25) (layer F.Cu) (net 10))
 (segment (start 97.155 42.545) (end 96.02363 42.545) (width 0.25) (layer F.Cu) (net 10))
 (segment (start 94.615 45.085) (end 97.155 45.085) (width 0.25) (layer F.Cu) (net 9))
 (segment (start 110.744 35.407) (end 110.744 36.007) (width 0.25) (layer F.Cu) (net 1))
 (segment (start 110.29399 34.95699) (end 110.744 35.407) (width 0.25) (layer F.Cu) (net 1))
 (segment (start 97.932011 34.95699) (end 110.29399 34.95699) (width 0.25) (layer F.Cu) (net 1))
 (segment (start 96.059001 36.83) (end 97.932011 34.95699) (width 0.25) (layer F.Cu) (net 1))
 (segment (start 108.539 36.007) (end 108.839 36.007) (width 0.25) (layer F.Cu) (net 2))
 (segment (start 107.939 35.407) (end 108.539 36.007) (width 0.25) (layer F.Cu) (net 2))
 (segment (start 100.022001 35.407) (end 107.939 35.407) (width 0.25) (layer F.Cu) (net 2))
 (segment (start 98.599001 36.83) (end 100.022001 35.407) (width 0.25) (layer F.Cu) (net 2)))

